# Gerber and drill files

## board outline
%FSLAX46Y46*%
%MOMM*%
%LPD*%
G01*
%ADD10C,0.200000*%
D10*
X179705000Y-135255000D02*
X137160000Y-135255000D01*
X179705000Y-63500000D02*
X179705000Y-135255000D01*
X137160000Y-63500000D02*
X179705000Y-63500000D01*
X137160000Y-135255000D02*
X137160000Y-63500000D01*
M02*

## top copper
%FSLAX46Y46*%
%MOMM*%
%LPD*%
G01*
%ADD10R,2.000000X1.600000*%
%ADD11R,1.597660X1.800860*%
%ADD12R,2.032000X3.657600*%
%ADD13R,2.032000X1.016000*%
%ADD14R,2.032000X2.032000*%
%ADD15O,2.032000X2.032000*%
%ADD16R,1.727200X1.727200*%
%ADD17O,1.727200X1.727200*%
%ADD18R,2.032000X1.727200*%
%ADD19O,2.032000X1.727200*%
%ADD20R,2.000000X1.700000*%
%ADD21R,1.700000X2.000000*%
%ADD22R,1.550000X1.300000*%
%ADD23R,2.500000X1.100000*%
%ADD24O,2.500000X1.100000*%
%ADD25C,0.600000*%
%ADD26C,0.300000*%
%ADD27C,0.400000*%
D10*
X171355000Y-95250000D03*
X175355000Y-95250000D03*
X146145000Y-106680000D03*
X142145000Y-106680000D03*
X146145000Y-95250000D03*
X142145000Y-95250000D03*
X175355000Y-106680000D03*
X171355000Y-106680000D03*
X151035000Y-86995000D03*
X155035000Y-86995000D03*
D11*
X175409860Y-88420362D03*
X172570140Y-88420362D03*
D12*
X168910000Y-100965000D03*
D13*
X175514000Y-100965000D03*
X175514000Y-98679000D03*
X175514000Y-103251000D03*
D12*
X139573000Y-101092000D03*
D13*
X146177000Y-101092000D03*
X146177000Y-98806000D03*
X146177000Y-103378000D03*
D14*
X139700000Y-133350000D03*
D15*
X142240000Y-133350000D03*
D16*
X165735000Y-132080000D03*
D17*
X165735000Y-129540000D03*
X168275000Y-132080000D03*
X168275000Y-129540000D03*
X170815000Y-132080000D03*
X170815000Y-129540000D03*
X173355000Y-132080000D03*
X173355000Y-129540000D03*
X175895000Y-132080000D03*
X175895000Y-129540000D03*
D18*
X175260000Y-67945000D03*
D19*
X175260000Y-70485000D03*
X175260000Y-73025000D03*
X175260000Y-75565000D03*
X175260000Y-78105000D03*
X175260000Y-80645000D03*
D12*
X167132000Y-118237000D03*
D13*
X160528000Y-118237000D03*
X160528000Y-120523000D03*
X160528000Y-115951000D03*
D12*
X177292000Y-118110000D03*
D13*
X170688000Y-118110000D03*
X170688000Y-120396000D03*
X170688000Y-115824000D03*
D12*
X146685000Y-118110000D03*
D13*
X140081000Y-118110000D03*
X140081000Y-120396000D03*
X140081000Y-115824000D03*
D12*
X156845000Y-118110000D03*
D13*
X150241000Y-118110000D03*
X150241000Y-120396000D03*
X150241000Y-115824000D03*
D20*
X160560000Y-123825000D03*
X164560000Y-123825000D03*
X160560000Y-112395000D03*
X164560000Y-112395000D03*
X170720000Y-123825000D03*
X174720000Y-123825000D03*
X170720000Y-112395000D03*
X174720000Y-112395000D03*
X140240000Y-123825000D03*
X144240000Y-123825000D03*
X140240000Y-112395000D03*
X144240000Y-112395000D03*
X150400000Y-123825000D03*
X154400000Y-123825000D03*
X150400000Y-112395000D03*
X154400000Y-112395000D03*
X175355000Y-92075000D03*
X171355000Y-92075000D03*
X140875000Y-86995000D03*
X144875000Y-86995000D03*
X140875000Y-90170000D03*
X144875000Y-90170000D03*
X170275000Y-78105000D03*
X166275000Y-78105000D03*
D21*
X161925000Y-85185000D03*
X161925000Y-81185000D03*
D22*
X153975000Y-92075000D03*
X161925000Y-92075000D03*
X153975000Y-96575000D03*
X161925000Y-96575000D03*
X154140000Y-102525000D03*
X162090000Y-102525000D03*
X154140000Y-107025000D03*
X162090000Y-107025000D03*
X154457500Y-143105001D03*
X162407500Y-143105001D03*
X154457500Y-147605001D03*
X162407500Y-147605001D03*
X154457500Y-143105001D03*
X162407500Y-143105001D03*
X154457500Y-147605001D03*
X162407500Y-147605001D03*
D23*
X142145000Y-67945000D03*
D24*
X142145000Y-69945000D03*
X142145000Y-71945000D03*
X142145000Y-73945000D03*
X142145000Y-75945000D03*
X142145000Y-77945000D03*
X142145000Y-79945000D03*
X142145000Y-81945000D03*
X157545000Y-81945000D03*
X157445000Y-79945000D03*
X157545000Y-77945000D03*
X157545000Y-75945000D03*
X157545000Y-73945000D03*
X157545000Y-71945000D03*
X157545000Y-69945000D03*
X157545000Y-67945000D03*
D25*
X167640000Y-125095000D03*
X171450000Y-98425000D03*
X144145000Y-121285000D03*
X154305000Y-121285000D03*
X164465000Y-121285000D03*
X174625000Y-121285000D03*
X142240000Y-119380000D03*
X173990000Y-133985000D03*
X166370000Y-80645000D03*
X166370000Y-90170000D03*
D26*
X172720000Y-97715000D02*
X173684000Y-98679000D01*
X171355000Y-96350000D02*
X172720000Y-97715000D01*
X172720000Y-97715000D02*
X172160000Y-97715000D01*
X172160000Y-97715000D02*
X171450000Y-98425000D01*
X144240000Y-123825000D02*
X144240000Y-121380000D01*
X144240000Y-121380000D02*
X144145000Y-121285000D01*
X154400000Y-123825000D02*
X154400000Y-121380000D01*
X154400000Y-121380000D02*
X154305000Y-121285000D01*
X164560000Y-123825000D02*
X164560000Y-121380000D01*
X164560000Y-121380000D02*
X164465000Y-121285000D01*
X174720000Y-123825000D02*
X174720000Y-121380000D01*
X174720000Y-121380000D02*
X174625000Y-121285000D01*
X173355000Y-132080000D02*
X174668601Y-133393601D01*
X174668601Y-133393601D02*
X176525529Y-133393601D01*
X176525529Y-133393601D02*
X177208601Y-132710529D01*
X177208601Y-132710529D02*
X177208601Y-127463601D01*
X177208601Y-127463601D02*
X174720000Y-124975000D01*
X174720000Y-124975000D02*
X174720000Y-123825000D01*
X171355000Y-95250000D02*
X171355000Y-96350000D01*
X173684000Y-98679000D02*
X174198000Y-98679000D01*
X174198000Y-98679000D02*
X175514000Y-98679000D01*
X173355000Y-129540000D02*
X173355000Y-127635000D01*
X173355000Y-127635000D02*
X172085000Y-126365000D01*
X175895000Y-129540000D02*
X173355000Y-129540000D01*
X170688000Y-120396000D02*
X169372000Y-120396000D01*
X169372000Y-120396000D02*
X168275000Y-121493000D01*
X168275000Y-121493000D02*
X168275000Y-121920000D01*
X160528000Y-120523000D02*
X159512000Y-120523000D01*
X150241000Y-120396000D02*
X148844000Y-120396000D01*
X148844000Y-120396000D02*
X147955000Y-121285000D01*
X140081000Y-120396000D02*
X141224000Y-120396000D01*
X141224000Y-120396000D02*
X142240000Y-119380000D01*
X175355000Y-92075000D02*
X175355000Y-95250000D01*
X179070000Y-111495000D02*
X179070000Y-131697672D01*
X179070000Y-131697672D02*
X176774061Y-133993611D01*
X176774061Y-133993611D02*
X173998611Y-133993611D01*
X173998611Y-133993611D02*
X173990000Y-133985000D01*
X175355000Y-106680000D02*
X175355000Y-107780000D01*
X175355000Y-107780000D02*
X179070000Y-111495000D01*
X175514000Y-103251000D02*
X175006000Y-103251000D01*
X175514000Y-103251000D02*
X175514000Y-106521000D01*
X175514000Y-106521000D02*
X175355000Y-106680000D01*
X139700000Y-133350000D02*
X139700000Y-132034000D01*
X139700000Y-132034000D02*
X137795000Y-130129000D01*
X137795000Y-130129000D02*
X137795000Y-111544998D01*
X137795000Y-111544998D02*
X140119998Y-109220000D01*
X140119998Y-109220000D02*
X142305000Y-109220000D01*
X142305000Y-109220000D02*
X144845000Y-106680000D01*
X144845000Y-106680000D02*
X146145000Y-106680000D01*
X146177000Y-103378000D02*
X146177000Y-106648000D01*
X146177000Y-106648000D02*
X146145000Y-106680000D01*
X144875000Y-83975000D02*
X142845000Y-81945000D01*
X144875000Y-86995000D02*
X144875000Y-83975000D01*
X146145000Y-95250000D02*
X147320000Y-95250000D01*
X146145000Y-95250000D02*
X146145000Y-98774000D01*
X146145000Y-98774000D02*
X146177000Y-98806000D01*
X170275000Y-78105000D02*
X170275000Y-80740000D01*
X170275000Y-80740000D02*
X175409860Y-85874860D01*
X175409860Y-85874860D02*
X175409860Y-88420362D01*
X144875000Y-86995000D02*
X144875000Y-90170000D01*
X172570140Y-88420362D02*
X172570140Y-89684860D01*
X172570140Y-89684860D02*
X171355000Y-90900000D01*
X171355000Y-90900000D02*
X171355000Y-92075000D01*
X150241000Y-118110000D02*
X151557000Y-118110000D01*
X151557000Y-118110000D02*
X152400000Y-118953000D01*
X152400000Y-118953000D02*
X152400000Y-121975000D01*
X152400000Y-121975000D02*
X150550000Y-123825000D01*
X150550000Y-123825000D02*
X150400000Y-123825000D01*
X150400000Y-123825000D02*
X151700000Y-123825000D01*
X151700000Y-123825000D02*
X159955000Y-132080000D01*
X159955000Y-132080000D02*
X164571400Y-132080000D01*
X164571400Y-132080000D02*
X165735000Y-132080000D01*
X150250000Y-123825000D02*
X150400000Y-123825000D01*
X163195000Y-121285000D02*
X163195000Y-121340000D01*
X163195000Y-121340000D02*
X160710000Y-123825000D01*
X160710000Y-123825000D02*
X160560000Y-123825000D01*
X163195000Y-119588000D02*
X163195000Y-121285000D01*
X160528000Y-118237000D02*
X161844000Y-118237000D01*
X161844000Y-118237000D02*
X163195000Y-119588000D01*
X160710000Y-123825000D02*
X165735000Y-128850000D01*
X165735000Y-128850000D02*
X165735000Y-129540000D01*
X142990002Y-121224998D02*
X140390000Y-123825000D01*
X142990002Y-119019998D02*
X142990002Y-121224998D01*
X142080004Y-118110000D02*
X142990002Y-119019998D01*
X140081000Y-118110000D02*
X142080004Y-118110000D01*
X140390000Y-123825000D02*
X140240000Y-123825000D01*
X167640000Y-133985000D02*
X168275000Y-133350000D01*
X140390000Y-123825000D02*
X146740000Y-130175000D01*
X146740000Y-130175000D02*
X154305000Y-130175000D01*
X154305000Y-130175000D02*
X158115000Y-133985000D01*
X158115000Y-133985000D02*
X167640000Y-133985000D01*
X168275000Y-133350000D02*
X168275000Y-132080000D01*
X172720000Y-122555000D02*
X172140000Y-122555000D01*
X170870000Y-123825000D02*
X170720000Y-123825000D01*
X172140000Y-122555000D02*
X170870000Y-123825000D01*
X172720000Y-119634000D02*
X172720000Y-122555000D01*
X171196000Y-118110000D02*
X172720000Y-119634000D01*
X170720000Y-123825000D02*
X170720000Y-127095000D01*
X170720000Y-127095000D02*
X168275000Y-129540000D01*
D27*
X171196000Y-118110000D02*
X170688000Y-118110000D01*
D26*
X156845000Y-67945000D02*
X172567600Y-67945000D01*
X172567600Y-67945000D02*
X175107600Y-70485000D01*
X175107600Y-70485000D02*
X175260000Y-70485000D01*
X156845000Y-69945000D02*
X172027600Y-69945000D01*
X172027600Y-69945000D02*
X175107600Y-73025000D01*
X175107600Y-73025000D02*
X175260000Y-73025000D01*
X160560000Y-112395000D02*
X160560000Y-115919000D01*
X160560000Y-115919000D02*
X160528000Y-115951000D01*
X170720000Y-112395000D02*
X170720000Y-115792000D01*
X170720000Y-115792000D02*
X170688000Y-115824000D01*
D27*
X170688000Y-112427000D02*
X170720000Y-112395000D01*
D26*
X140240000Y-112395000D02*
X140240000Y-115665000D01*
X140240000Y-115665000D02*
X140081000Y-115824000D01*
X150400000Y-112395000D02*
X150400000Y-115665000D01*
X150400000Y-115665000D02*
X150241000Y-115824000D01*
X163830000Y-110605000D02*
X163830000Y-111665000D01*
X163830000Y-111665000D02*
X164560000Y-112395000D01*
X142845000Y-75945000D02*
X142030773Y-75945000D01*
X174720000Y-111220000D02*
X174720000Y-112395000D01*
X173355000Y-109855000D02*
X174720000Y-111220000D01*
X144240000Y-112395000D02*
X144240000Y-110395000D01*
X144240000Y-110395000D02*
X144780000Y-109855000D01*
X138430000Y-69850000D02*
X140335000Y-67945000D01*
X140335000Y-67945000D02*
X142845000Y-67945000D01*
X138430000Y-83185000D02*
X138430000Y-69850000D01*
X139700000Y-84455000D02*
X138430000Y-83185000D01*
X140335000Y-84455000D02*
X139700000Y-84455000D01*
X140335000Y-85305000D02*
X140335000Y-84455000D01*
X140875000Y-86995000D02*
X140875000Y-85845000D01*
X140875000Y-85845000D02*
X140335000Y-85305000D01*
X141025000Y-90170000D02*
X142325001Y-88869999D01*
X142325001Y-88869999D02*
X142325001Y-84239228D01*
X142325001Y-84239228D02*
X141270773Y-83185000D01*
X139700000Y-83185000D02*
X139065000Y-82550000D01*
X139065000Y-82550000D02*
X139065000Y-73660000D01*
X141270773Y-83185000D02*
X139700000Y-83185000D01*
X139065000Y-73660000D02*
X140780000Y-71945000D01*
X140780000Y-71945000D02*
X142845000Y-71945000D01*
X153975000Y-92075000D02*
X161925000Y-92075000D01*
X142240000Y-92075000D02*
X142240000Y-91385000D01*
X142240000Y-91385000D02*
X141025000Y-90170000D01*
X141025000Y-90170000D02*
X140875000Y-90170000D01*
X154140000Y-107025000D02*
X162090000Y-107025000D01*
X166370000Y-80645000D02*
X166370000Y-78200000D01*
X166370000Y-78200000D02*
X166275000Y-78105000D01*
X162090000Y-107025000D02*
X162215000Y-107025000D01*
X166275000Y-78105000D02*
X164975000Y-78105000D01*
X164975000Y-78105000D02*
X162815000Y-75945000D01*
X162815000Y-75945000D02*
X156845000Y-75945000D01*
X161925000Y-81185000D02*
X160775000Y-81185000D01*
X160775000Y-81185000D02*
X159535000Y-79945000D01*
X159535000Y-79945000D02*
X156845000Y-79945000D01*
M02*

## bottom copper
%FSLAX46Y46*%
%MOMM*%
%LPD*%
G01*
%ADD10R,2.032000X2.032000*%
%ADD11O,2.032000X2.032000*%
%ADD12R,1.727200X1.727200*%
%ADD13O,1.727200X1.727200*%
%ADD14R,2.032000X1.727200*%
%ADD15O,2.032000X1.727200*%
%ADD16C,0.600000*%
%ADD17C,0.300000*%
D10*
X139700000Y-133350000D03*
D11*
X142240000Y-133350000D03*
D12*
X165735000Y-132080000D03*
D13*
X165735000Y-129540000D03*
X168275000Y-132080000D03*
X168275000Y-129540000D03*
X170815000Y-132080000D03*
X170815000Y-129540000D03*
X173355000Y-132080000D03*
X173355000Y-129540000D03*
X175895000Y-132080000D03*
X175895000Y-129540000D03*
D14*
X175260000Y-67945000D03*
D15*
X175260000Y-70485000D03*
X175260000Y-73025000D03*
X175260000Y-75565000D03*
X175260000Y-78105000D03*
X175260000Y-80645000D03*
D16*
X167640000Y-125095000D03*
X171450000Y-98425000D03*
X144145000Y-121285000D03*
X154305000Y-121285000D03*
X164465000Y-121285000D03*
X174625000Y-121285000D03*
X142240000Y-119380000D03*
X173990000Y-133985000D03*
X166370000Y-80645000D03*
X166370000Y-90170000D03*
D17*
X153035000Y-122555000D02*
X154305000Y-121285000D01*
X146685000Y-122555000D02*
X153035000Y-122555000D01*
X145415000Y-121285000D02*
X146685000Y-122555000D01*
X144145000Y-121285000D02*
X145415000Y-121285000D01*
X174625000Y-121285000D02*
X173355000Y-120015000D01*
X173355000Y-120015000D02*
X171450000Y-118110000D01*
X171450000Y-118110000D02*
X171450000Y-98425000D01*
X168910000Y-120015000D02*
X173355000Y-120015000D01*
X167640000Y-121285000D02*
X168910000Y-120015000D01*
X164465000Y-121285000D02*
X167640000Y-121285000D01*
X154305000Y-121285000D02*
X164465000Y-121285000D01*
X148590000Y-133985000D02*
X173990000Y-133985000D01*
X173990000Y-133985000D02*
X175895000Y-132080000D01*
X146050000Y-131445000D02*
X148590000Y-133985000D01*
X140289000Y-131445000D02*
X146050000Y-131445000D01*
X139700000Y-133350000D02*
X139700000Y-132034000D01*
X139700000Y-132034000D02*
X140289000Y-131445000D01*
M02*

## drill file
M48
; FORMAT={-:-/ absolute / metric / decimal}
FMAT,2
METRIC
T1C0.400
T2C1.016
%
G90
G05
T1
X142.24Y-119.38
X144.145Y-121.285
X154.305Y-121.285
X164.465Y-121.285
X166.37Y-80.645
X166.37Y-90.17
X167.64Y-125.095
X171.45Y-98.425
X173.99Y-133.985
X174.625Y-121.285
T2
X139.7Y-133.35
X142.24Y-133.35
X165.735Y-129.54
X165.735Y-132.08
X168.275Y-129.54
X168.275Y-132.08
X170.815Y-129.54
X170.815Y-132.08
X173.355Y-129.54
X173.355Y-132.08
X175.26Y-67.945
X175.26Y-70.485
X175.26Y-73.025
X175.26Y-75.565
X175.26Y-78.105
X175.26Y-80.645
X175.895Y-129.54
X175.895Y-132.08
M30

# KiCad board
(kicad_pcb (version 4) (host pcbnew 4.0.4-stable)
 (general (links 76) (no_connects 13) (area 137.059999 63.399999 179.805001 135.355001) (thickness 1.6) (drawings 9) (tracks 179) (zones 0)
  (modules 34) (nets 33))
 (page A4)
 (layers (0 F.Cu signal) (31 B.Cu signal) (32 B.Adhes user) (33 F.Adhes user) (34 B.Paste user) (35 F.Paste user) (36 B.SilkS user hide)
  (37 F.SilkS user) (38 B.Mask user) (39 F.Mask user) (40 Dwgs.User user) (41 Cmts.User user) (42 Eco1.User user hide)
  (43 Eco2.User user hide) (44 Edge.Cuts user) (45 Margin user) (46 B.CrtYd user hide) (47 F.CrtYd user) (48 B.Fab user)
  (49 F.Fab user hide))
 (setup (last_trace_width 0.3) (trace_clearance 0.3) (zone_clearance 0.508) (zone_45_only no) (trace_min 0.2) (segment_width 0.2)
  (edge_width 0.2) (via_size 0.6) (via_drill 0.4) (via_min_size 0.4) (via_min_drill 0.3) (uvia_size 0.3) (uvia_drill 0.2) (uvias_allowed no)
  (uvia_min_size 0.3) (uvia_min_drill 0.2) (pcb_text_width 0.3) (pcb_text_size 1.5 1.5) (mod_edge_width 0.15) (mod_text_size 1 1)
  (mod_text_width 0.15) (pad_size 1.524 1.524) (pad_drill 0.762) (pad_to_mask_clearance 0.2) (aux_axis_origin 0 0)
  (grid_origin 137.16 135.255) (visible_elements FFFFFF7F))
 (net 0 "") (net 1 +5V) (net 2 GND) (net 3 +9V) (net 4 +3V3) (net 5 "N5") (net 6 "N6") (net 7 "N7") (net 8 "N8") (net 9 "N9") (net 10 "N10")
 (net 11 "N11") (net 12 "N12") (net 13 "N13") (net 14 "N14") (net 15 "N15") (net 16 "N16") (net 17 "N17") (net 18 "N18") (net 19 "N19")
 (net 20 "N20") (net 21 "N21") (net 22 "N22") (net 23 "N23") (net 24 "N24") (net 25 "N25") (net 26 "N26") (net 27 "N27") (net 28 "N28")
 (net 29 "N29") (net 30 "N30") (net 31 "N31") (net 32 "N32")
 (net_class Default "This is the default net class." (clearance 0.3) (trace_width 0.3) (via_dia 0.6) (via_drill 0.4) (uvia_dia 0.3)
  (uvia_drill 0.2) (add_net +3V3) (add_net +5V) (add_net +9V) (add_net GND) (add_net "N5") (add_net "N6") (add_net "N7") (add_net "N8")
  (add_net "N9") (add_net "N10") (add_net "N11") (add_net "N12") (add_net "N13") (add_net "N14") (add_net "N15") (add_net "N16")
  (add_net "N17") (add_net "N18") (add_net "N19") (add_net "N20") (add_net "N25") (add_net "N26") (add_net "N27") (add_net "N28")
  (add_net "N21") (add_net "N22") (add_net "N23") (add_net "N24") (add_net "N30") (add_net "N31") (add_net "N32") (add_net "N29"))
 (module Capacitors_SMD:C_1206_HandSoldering (layer F.Cu) (at 173.355 95.25)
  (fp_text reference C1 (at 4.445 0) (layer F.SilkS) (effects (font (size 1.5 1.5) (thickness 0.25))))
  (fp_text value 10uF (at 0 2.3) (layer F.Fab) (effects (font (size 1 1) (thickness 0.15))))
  (pad 1 smd rect (at -2 0) (size 2 1.6) (layers F.Cu F.Paste F.Mask) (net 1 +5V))
  (pad 2 smd rect (at 2 0) (size 2 1.6) (layers F.Cu F.Paste F.Mask) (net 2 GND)))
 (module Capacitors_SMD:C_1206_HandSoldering (layer F.Cu) (at 144.145 106.68 180)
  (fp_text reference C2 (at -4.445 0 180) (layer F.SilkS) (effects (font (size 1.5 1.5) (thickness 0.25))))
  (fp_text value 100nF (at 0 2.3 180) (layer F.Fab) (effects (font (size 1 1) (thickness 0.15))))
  (pad 1 smd rect (at -2 0 180) (size 2 1.6) (layers F.Cu F.Paste F.Mask) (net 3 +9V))
  (pad 2 smd rect (at 2 0 180) (size 2 1.6) (layers F.Cu F.Paste F.Mask) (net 2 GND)))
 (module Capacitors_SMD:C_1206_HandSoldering (layer F.Cu) (at 144.145 95.25 180)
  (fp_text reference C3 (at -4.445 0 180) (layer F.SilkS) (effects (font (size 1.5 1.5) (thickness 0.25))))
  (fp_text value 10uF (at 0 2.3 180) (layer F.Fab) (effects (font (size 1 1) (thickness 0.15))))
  (pad 1 smd rect (at -2 0 180) (size 2 1.6) (layers F.Cu F.Paste F.Mask) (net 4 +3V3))
  (pad 2 smd rect (at 2 0 180) (size 2 1.6) (layers F.Cu F.Paste F.Mask) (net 2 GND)))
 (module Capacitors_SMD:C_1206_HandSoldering (layer F.Cu) (at 173.355 106.68 180)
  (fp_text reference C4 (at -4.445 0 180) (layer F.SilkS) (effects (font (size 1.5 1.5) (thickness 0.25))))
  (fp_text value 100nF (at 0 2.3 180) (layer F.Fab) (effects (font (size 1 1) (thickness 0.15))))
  (pad 1 smd rect (at -2 0 180) (size 2 1.6) (layers F.Cu F.Paste F.Mask) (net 3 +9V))
  (pad 2 smd rect (at 2 0 180) (size 2 1.6) (layers F.Cu F.Paste F.Mask) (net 2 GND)))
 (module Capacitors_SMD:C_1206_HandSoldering (layer F.Cu) (at 153.035 86.995)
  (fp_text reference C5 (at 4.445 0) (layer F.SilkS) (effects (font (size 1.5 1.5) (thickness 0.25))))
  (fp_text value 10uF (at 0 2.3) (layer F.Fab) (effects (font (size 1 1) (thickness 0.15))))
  (pad 1 smd rect (at -2 0) (size 2 1.6) (layers F.Cu F.Paste F.Mask) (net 4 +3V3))
  (pad 2 smd rect (at 2 0) (size 2 1.6) (layers F.Cu F.Paste F.Mask) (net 2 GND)))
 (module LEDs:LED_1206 (layer F.Cu) (at 173.99 88.420362)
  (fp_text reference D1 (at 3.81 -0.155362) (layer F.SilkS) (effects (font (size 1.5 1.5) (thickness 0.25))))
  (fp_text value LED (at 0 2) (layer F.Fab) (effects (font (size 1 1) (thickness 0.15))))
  (pad 2 smd rect (at 1.41986 0 180) (size 1.59766 1.80086) (layers F.Cu F.Paste F.Mask) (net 4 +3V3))
  (pad 1 smd rect (at -1.41986 0 180) (size 1.59766 1.80086) (layers F.Cu F.Paste F.Mask) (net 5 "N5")))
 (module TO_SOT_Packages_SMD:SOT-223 (layer F.Cu) (at 172.212 100.965 90)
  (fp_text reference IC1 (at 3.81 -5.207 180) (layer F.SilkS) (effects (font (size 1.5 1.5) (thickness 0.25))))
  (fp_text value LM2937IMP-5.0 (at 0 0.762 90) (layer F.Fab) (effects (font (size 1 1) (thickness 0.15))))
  (pad 4 smd rect (at 0 -3.302 90) (size 3.6576 2.032) (layers F.Cu F.Paste F.Mask) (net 2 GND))
  (pad 2 smd rect (at 0 3.302 90) (size 1.016 2.032) (layers F.Cu F.Paste F.Mask) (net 2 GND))
  (pad 3 smd rect (at 2.286 3.302 90) (size 1.016 2.032) (layers F.Cu F.Paste F.Mask) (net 1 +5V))
  (pad 1 smd rect (at -2.286 3.302 90) (size 1.016 2.032) (layers F.Cu F.Paste F.Mask) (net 3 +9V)))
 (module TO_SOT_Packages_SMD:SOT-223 (layer F.Cu) (at 142.875 101.092 90)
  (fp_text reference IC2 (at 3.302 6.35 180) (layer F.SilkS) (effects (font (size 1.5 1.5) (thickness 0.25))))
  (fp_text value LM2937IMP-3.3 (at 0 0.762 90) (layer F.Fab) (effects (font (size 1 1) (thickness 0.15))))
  (pad 4 smd rect (at 0 -3.302 90) (size 3.6576 2.032) (layers F.Cu F.Paste F.Mask) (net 2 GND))
  (pad 2 smd rect (at 0 3.302 90) (size 1.016 2.032) (layers F.Cu F.Paste F.Mask) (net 2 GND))
  (pad 3 smd rect (at 2.286 3.302 90) (size 1.016 2.032) (layers F.Cu F.Paste F.Mask) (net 4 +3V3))
  (pad 1 smd rect (at -2.286 3.302 90) (size 1.016 2.032) (layers F.Cu F.Paste F.Mask) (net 3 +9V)))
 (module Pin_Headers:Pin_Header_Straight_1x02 (layer F.Cu) (at 139.7 133.35 90)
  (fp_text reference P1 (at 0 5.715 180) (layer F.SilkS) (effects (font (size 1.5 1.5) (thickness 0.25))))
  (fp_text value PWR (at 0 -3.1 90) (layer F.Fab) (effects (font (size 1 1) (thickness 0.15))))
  (pad 1 thru_hole rect (at 0 0 90) (size 2.032 2.032) (drill 1.016) (layers *.Cu *.Mask) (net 3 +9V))
  (pad 2 thru_hole oval (at 0 2.54 90) (size 2.032 2.032) (drill 1.016) (layers *.Cu *.Mask) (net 2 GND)))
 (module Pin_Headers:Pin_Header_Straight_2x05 (layer F.Cu) (at 165.735 132.08 90)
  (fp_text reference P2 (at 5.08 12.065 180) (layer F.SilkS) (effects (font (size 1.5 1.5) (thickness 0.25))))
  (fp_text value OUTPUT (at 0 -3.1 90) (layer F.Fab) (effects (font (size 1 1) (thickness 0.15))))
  (pad 1 thru_hole rect (at 0 0 90) (size 1.7272 1.7272) (drill 1.016) (layers *.Cu *.Mask) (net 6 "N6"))
  (pad 2 thru_hole oval (at 2.54 0 90) (size 1.7272 1.7272) (drill 1.016) (layers *.Cu *.Mask) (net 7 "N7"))
  (pad 3 thru_hole oval (at 0 2.54 90) (size 1.7272 1.7272) (drill 1.016) (layers *.Cu *.Mask) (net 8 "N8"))
  (pad 4 thru_hole oval (at 2.54 2.54 90) (size 1.7272 1.7272) (drill 1.016) (layers *.Cu *.Mask) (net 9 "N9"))
  (pad 5 thru_hole oval (at 0 5.08 90) (size 1.7272 1.7272) (drill 1.016) (layers *.Cu *.Mask) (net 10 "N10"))
  (pad 6 thru_hole oval (at 2.54 5.08 90) (size 1.7272 1.7272) (drill 1.016) (layers *.Cu *.Mask) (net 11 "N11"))
  (pad 7 thru_hole oval (at 0 7.62 90) (size 1.7272 1.7272) (drill 1.016) (layers *.Cu *.Mask) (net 1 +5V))
  (pad 8 thru_hole oval (at 2.54 7.62 90) (size 1.7272 1.7272) (drill 1.016) (layers *.Cu *.Mask) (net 2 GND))
  (pad 9 thru_hole oval (at 0 10.16 90) (size 1.7272 1.7272) (drill 1.016) (layers *.Cu *.Mask) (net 3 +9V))
  (pad 10 thru_hole oval (at 2.54 10.16 90) (size 1.7272 1.7272) (drill 1.016) (layers *.Cu *.Mask) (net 2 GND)))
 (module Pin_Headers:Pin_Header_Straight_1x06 (layer F.Cu) (at 175.26 67.945)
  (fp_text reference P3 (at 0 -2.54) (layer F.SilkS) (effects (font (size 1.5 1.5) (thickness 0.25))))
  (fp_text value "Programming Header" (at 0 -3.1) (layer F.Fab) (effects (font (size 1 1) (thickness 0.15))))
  (pad 1 thru_hole rect (at 0 0) (size 2.032 1.7272) (drill 1.016) (layers *.Cu *.Mask) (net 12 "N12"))
  (pad 2 thru_hole oval (at 0 2.54) (size 2.032 1.7272) (drill 1.016) (layers *.Cu *.Mask) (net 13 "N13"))
  (pad 3 thru_hole oval (at 0 5.08) (size 2.032 1.7272) (drill 1.016) (layers *.Cu *.Mask) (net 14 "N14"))
  (pad 4 thru_hole oval (at 0 7.62) (size 2.032 1.7272) (drill 1.016) (layers *.Cu *.Mask) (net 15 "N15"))
  (pad 5 thru_hole oval (at 0 10.16) (size 2.032 1.7272) (drill 1.016) (layers *.Cu *.Mask) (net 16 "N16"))
  (pad 6 thru_hole oval (at 0 12.7) (size 2.032 1.7272) (drill 1.016) (layers *.Cu *.Mask) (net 2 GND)))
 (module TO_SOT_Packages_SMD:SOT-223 (layer F.Cu) (at 163.83 118.237 270)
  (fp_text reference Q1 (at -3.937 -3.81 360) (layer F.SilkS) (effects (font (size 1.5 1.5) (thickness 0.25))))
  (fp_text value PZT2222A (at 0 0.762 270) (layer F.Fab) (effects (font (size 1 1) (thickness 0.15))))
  (pad 4 smd rect (at 0 -3.302 270) (size 3.6576 2.032) (layers F.Cu F.Paste F.Mask))
  (pad 2 smd rect (at 0 3.302 270) (size 1.016 2.032) (layers F.Cu F.Paste F.Mask) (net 7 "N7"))
  (pad 3 smd rect (at 2.286 3.302 270) (size 1.016 2.032) (layers F.Cu F.Paste F.Mask) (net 2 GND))
  (pad 1 smd rect (at -2.286 3.302 270) (size 1.016 2.032) (layers F.Cu F.Paste F.Mask) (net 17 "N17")))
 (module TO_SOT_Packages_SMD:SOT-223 (layer F.Cu) (at 173.99 118.11 270)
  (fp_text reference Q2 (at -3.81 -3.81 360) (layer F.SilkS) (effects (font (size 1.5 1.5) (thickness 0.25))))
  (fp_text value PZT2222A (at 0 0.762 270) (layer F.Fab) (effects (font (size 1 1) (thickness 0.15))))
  (pad 4 smd rect (at 0 -3.302 270) (size 3.6576 2.032) (layers F.Cu F.Paste F.Mask))
  (pad 2 smd rect (at 0 3.302 270) (size 1.016 2.032) (layers F.Cu F.Paste F.Mask) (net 9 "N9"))
  (pad 3 smd rect (at 2.286 3.302 270) (size 1.016 2.032) (layers F.Cu F.Paste F.Mask) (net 2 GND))
  (pad 1 smd rect (at -2.286 3.302 270) (size 1.016 2.032) (layers F.Cu F.Paste F.Mask) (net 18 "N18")))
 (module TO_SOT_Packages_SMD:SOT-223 (layer F.Cu) (at 143.383 118.11 270)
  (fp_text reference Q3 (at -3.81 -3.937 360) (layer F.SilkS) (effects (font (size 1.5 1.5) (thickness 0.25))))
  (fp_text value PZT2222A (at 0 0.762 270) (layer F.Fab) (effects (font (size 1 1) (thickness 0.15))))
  (pad 4 smd rect (at 0 -3.302 270) (size 3.6576 2.032) (layers F.Cu F.Paste F.Mask))
  (pad 2 smd rect (at 0 3.302 270) (size 1.016 2.032) (layers F.Cu F.Paste F.Mask) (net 8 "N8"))
  (pad 3 smd rect (at 2.286 3.302 270) (size 1.016 2.032) (layers F.Cu F.Paste F.Mask) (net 2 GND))
  (pad 1 smd rect (at -2.286 3.302 270) (size 1.016 2.032) (layers F.Cu F.Paste F.Mask) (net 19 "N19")))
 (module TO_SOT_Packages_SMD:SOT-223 (layer F.Cu) (at 153.543 118.11 270)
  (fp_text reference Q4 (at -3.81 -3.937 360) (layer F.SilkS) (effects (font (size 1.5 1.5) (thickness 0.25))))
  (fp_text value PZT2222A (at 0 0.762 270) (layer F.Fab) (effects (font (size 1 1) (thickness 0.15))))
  (pad 4 smd rect (at 0 -3.302 270) (size 3.6576 2.032) (layers F.Cu F.Paste F.Mask))
  (pad 2 smd rect (at 0 3.302 270) (size 1.016 2.032) (layers F.Cu F.Paste F.Mask) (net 6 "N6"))
  (pad 3 smd rect (at 2.286 3.302 270) (size 1.016 2.032) (layers F.Cu F.Paste F.Mask) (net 2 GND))
  (pad 1 smd rect (at -2.286 3.302 270) (size 1.016 2.032) (layers F.Cu F.Paste F.Mask) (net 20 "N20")))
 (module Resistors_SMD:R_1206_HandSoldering (layer F.Cu) (at 162.56 123.825)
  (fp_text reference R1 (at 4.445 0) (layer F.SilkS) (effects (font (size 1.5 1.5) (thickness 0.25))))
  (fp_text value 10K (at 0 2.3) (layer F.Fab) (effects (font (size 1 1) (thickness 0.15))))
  (pad 1 smd rect (at -2 0) (size 2 1.7) (layers F.Cu F.Paste F.Mask) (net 7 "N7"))
  (pad 2 smd rect (at 2 0) (size 2 1.7) (layers F.Cu F.Paste F.Mask) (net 1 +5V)))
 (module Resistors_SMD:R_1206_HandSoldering (layer F.Cu) (at 162.56 112.395)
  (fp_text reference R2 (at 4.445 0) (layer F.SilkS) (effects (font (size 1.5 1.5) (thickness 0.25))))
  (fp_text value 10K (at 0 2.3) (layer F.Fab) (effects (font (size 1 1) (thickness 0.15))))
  (pad 1 smd rect (at -2 0) (size 2 1.7) (layers F.Cu F.Paste F.Mask) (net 17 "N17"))
  (pad 2 smd rect (at 2 0) (size 2 1.7) (layers F.Cu F.Paste F.Mask) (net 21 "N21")))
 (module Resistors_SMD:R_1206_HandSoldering (layer F.Cu) (at 172.72 123.825)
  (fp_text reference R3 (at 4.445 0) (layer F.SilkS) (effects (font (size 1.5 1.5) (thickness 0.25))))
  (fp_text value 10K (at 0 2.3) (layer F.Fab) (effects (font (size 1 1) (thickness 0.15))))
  (pad 1 smd rect (at -2 0) (size 2 1.7) (layers F.Cu F.Paste F.Mask) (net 9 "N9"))
  (pad 2 smd rect (at 2 0) (size 2 1.7) (layers F.Cu F.Paste F.Mask) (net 1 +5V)))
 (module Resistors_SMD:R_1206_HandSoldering (layer F.Cu) (at 172.72 112.395)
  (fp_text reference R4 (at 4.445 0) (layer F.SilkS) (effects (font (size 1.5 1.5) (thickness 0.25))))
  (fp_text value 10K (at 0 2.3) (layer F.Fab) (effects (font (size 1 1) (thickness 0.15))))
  (pad 1 smd rect (at -2 0) (size 2 1.7) (layers F.Cu F.Paste F.Mask) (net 18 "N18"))
  (pad 2 smd rect (at 2 0) (size 2 1.7) (layers F.Cu F.Paste F.Mask) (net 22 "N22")))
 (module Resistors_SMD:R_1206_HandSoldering (layer F.Cu) (at 142.24 123.825)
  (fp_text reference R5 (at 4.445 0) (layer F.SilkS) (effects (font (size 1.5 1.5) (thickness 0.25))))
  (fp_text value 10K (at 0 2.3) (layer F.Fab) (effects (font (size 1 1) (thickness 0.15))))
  (pad 1 smd rect (at -2 0) (size 2 1.7) (layers F.Cu F.Paste F.Mask) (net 8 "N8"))
  (pad 2 smd rect (at 2 0) (size 2 1.7) (layers F.Cu F.Paste F.Mask) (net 1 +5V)))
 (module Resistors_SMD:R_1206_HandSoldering (layer F.Cu) (at 142.24 112.395)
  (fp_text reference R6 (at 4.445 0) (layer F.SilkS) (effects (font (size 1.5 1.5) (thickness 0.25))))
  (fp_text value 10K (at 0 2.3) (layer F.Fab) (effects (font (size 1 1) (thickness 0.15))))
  (pad 1 smd rect (at -2 0) (size 2 1.7) (layers F.Cu F.Paste F.Mask) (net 19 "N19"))
  (pad 2 smd rect (at 2 0) (size 2 1.7) (layers F.Cu F.Paste F.Mask) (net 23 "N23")))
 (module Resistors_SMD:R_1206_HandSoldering (layer F.Cu) (at 152.4 123.825)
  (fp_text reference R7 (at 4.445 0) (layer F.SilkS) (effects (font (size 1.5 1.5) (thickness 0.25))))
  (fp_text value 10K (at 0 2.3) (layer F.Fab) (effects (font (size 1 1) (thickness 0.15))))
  (pad 1 smd rect (at -2 0) (size 2 1.7) (layers F.Cu F.Paste F.Mask) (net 6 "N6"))
  (pad 2 smd rect (at 2 0) (size 2 1.7) (layers F.Cu F.Paste F.Mask) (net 1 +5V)))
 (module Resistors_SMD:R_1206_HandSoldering (layer F.Cu) (at 152.4 112.395)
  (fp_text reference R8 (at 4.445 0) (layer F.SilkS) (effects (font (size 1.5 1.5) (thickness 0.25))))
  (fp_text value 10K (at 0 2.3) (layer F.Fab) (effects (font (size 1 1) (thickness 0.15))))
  (pad 1 smd rect (at -2 0) (size 2 1.7) (layers F.Cu F.Paste F.Mask) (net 20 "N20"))
  (pad 2 smd rect (at 2 0) (size 2 1.7) (layers F.Cu F.Paste F.Mask) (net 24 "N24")))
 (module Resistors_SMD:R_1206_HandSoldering (layer F.Cu) (at 173.355 92.075 180)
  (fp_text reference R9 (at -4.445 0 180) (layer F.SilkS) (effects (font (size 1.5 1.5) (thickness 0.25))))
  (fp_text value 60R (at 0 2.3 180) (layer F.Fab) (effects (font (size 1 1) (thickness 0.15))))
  (pad 1 smd rect (at -2 0 180) (size 2 1.7) (layers F.Cu F.Paste F.Mask) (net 2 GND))
  (pad 2 smd rect (at 2 0 180) (size 2 1.7) (layers F.Cu F.Paste F.Mask) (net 5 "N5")))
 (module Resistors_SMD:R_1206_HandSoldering (layer F.Cu) (at 142.875 86.995)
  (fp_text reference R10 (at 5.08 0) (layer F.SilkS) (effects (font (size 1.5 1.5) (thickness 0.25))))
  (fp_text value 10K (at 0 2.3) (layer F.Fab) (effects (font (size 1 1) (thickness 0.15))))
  (pad 1 smd rect (at -2 0) (size 2 1.7) (layers F.Cu F.Paste F.Mask) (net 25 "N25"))
  (pad 2 smd rect (at 2 0) (size 2 1.7) (layers F.Cu F.Paste F.Mask) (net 4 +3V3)))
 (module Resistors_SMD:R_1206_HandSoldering (layer F.Cu) (at 142.875 90.17)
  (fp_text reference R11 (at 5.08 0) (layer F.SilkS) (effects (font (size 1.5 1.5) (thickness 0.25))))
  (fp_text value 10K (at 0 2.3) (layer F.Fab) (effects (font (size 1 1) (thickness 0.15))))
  (pad 1 smd rect (at -2 0) (size 2 1.7) (layers F.Cu F.Paste F.Mask) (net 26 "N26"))
  (pad 2 smd rect (at 2 0) (size 2 1.7) (layers F.Cu F.Paste F.Mask) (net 4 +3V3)))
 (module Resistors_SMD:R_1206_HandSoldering (layer F.Cu) (at 168.275 78.105 180)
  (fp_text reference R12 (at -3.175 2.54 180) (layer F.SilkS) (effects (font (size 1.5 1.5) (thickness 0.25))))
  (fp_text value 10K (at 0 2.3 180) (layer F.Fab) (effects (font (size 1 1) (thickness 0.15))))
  (pad 1 smd rect (at -2 0 180) (size 2 1.7) (layers F.Cu F.Paste F.Mask) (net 4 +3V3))
  (pad 2 smd rect (at 2 0 180) (size 2 1.7) (layers F.Cu F.Paste F.Mask) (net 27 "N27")))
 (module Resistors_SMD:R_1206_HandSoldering (layer F.Cu) (at 161.925 83.185 90)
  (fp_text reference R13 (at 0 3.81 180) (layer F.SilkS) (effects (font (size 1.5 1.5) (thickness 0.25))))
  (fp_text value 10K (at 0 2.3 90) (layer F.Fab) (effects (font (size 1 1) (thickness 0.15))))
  (pad 1 smd rect (at -2 0 90) (size 2 1.7) (layers F.Cu F.Paste F.Mask) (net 2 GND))
  (pad 2 smd rect (at 2 0 90) (size 2 1.7) (layers F.Cu F.Paste F.Mask) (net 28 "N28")))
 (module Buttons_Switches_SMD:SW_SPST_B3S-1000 (layer F.Cu) (at 157.95 94.325)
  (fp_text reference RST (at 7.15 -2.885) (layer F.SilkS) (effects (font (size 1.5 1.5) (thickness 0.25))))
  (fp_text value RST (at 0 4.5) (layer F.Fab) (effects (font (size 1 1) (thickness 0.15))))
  (pad 1 smd rect (at -3.975 -2.25) (size 1.55 1.3) (layers F.Cu F.Paste F.Mask) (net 26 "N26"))
  (pad 1 smd rect (at 3.975 -2.25) (size 1.55 1.3) (layers F.Cu F.Paste F.Mask) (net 26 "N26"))
  (pad 2 smd rect (at -3.975 2.25) (size 1.55 1.3) (layers F.Cu F.Paste F.Mask) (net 2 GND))
  (pad 2 smd rect (at 3.975 2.25) (size 1.55 1.3) (layers F.Cu F.Paste F.Mask) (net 2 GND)))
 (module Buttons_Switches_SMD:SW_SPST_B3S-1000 (layer F.Cu) (at 158.115 104.775)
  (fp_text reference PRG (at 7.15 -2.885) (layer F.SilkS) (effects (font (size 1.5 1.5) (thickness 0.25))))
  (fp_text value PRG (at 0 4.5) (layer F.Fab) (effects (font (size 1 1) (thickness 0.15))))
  (pad 1 smd rect (at -3.975 -2.25) (size 1.55 1.3) (layers F.Cu F.Paste F.Mask) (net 2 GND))
  (pad 1 smd rect (at 3.975 -2.25) (size 1.55 1.3) (layers F.Cu F.Paste F.Mask) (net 2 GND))
  (pad 2 smd rect (at -3.975 2.25) (size 1.55 1.3) (layers F.Cu F.Paste F.Mask) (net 27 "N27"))
  (pad 2 smd rect (at 3.975 2.25) (size 1.55 1.3) (layers F.Cu F.Paste F.Mask) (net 27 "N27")))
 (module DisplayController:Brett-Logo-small (layer B.Cu) (at 165.735 119.38 270)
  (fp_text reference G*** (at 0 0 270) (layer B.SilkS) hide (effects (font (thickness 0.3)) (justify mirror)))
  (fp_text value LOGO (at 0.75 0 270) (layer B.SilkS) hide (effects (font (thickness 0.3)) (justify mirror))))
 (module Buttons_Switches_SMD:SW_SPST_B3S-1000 (layer F.Cu) (at 158.4325 145.355001)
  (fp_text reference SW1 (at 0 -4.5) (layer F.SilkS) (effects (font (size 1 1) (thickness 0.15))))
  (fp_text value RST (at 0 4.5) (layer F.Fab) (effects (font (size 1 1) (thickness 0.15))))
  (pad 1 smd rect (at -3.975 -2.25) (size 1.55 1.3) (layers F.Cu F.Paste F.Mask) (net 26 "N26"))
  (pad 1 smd rect (at 3.975 -2.25) (size 1.55 1.3) (layers F.Cu F.Paste F.Mask) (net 26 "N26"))
  (pad 2 smd rect (at -3.975 2.25) (size 1.55 1.3) (layers F.Cu F.Paste F.Mask) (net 2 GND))
  (pad 2 smd rect (at 3.975 2.25) (size 1.55 1.3) (layers F.Cu F.Paste F.Mask) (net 2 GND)))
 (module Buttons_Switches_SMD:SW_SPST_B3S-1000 (layer F.Cu) (at 158.4325 145.355001)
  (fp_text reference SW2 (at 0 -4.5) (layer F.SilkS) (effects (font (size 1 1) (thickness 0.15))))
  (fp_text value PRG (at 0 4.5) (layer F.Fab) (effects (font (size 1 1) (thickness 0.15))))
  (pad 1 smd rect (at -3.975 -2.25) (size 1.55 1.3) (layers F.Cu F.Paste F.Mask) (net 2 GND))
  (pad 1 smd rect (at 3.975 -2.25) (size 1.55 1.3) (layers F.Cu F.Paste F.Mask) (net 2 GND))
  (pad 2 smd rect (at -3.975 2.25) (size 1.55 1.3) (layers F.Cu F.Paste F.Mask) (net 27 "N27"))
  (pad 2 smd rect (at 3.975 2.25) (size 1.55 1.3) (layers F.Cu F.Paste F.Mask) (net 27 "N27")))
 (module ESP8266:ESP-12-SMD (layer F.Cu) (at 142.845 67.945)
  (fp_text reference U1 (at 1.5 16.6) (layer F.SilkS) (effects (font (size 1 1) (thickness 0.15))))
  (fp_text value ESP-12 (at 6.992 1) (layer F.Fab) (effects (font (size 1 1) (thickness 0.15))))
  (pad 1 smd rect (at 0 0) (size 2.5 1.1) (drill (offset -0.7 0)) (layers F.Cu F.Paste F.Mask) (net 25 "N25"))
  (pad 2 smd oval (at 0 2) (size 2.5 1.1) (drill (offset -0.7 0)) (layers F.Cu F.Paste F.Mask) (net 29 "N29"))
  (pad 3 smd oval (at 0 4) (size 2.5 1.1) (drill (offset -0.7 0)) (layers F.Cu F.Paste F.Mask) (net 26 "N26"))
  (pad 4 smd oval (at 0 6) (size 2.5 1.1) (drill (offset -0.7 0)) (layers F.Cu F.Paste F.Mask) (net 21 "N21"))
  (pad 5 smd oval (at 0 8) (size 2.5 1.1) (drill (offset -0.7 0)) (layers F.Cu F.Paste F.Mask) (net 22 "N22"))
  (pad 6 smd oval (at 0 10) (size 2.5 1.1) (drill (offset -0.7 0)) (layers F.Cu F.Paste F.Mask) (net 23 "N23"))
  (pad 7 smd oval (at 0 12) (size 2.5 1.1) (drill (offset -0.7 0)) (layers F.Cu F.Paste F.Mask) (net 24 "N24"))
  (pad 8 smd oval (at 0 14) (size 2.5 1.1) (drill (offset -0.7 0)) (layers F.Cu F.Paste F.Mask) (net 4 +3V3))
  (pad 9 smd oval (at 14 14) (size 2.5 1.1) (drill (offset 0.7 0)) (layers F.Cu F.Paste F.Mask) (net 2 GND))
  (pad 10 smd oval (at 14 12) (size 2.5 1.1) (drill (offset 0.6 0)) (layers F.Cu F.Paste F.Mask) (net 28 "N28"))
  (pad 11 smd oval (at 14 10) (size 2.5 1.1) (drill (offset 0.7 0)) (layers F.Cu F.Paste F.Mask) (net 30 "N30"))
  (pad 12 smd oval (at 14 8) (size 2.5 1.1) (drill (offset 0.7 0)) (layers F.Cu F.Paste F.Mask) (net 27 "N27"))
  (pad 13 smd oval (at 14 6) (size 2.5 1.1) (drill (offset 0.7 0)) (layers F.Cu F.Paste F.Mask) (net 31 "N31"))
  (pad 14 smd oval (at 14 4) (size 2.5 1.1) (drill (offset 0.7 0)) (layers F.Cu F.Paste F.Mask) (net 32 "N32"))
  (pad 15 smd oval (at 14 2) (size 2.5 1.1) (drill (offset 0.7 0)) (layers F.Cu F.Paste F.Mask) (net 14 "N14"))
  (pad 16 smd oval (at 14 0) (size 2.5 1.1) (drill (offset 0.7 0)) (layers F.Cu F.Paste F.Mask) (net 13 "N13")))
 (gr_line (start 179.705 135.255) (end 137.16 135.255) (layer Edge.Cuts) (width 0.2))
 (gr_line (start 179.705 63.5) (end 179.705 135.255) (layer Edge.Cuts) (width 0.2))
 (gr_line (start 137.16 63.5) (end 179.705 63.5) (layer Edge.Cuts) (width 0.2))
 (gr_line (start 137.16 135.255) (end 137.16 63.5) (layer Edge.Cuts) (width 0.2))
 (via (at 167.64 125.095) (size 0.6) (drill 0.4) (layers F.Cu B.Cu) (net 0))
 (segment (start 153.035 122.555) (end 154.305 121.285) (width 0.3) (layer B.Cu) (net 1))
 (segment (start 146.685 122.555) (end 153.035 122.555) (width 0.3) (layer B.Cu) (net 1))
 (segment (start 145.415 121.285) (end 146.685 122.555) (width 0.3) (layer B.Cu) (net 1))
 (segment (start 144.145 121.285) (end 145.415 121.285) (width 0.3) (layer B.Cu) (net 1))
 (segment (start 174.625 121.285) (end 173.355 120.015) (width 0.3) (layer B.Cu) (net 1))
 (segment (start 173.355 120.015) (end 171.45 118.11) (width 0.3) (layer B.Cu) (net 1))
 (segment (start 171.45 118.11) (end 171.45 98.425) (width 0.3) (layer B.Cu) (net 1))
 (segment (start 168.91 120.015) (end 173.355 120.015) (width 0.3) (layer B.Cu) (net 1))
 (segment (start 167.64 121.285) (end 168.91 120.015) (width 0.3) (layer B.Cu) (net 1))
 (segment (start 164.465 121.285) (end 167.64 121.285) (width 0.3) (layer B.Cu) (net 1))
 (segment (start 154.305 121.285) (end 164.465 121.285) (width 0.3) (layer B.Cu) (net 1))
 (segment (start 172.72 97.715) (end 173.684 98.679) (width 0.3) (layer F.Cu) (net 1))
 (segment (start 171.355 96.35) (end 172.72 97.715) (width 0.3) (layer F.Cu) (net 1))
 (segment (start 172.72 97.715) (end 172.16 97.715) (width 0.3) (layer F.Cu) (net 1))
 (segment (start 172.16 97.715) (end 171.45 98.425) (width 0.3) (layer F.Cu) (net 1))
 (via (at 171.45 98.425) (size 0.6) (drill 0.4) (layers F.Cu B.Cu) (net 1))
 (segment (start 144.24 123.825) (end 144.24 121.38) (width 0.3) (layer F.Cu) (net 1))
 (segment (start 144.24 121.38) (end 144.145 121.285) (width 0.3) (layer F.Cu) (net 1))
 (via (at 144.145 121.285) (size 0.6) (drill 0.4) (layers F.Cu B.Cu) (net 1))
 (segment (start 154.4 123.825) (end 154.4 121.38) (width 0.3) (layer F.Cu) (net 1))
 (segment (start 154.4 121.38) (end 154.305 121.285) (width 0.3) (layer F.Cu) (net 1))
 (via (at 154.305 121.285) (size 0.6) (drill 0.4) (layers F.Cu B.Cu) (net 1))
 (segment (start 164.56 123.825) (end 164.56 121.38) (width 0.3) (layer F.Cu) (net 1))
 (segment (start 164.56 121.38) (end 164.465 121.285) (width 0.3) (layer F.Cu) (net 1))
 (via (at 164.465 121.285) (size 0.6) (drill 0.4) (layers F.Cu B.Cu) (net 1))
 (segment (start 174.72 123.825) (end 174.72 121.38) (width 0.3) (layer F.Cu) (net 1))
 (segment (start 174.72 121.38) (end 174.625 121.285) (width 0.3) (layer F.Cu) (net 1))
 (via (at 174.625 121.285) (size 0.6) (drill 0.4) (layers F.Cu B.Cu) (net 1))
 (segment (start 173.355 132.08) (end 174.668601 133.393601) (width 0.3) (layer F.Cu) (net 1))
 (segment (start 174.668601 133.393601) (end 176.525529 133.393601) (width 0.3) (layer F.Cu) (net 1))
 (segment (start 176.525529 133.393601) (end 177.208601 132.710529) (width 0.3) (layer F.Cu) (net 1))
 (segment (start 177.208601 132.710529) (end 177.208601 127.463601) (width 0.3) (layer F.Cu) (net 1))
 (segment (start 177.208601 127.463601) (end 174.72 124.975) (width 0.3) (layer F.Cu) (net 1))
 (segment (start 174.72 124.975) (end 174.72 123.825) (width 0.3) (layer F.Cu) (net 1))
 (segment (start 171.355 95.25) (end 171.355 96.35) (width 0.3) (layer F.Cu) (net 1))
 (segment (start 173.684 98.679) (end 174.198 98.679) (width 0.3) (layer F.Cu) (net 1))
 (segment (start 174.198 98.679) (end 175.514 98.679) (width 0.3) (layer F.Cu) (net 1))
 (via (at 142.24 119.38) (size 0.6) (drill 0.4) (layers F.Cu B.Cu) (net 2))
 (segment (start 173.355 129.54) (end 173.355 127.635) (width 0.3) (layer F.Cu) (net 2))
 (segment (start 173.355 127.635) (end 172.085 126.365) (width 0.3) (layer F.Cu) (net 2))
 (segment (start 175.895 129.54) (end 173.355 129.54) (width 0.3) (layer F.Cu) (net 2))
 (segment (start 170.688 120.396) (end 169.372 120.396) (width 0.3) (layer F.Cu) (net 2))
 (segment (start 169.372 120.396) (end 168.275 121.493) (width 0.3) (layer F.Cu) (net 2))
 (segment (start 168.275 121.493) (end 168.275 121.92) (width 0.3) (layer F.Cu) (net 2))
 (segment (start 160.528 120.523) (end 159.512 120.523) (width 0.3) (layer F.Cu) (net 2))
 (segment (start 150.241 120.396) (end 148.844 120.396) (width 0.3) (layer F.Cu) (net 2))
 (segment (start 148.844 120.396) (end 147.955 121.285) (width 0.3) (layer F.Cu) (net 2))
 (segment (start 140.081 120.396) (end 141.224 120.396) (width 0.3) (layer F.Cu) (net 2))
 (segment (start 141.224 120.396) (end 142.24 119.38) (width 0.3) (layer F.Cu) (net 2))
 (segment (start 175.355 92.075) (end 175.355 95.25) (width 0.3) (layer F.Cu) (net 2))
 (segment (start 179.07 111.495) (end 179.07 131.697672) (width 0.3) (layer F.Cu) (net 3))
 (segment (start 179.07 131.697672) (end 176.774061 133.993611) (width 0.3) (layer F.Cu) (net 3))
 (segment (start 176.774061 133.993611) (end 173.998611 133.993611) (width 0.3) (layer F.Cu) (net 3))
 (segment (start 173.998611 133.993611) (end 173.99 133.985) (width 0.3) (layer F.Cu) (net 3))
 (via (at 173.99 133.985) (size 0.6) (drill 0.4) (layers F.Cu B.Cu) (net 3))
 (segment (start 175.355 106.68) (end 175.355 107.78) (width 0.3) (layer F.Cu) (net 3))
 (segment (start 175.355 107.78) (end 179.07 111.495) (width 0.3) (layer F.Cu) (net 3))
 (segment (start 175.514 103.251) (end 175.006 103.251) (width 0.3) (layer F.Cu) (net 3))
 (segment (start 175.514 103.251) (end 175.514 106.521) (width 0.3) (layer F.Cu) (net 3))
 (segment (start 175.514 106.521) (end 175.355 106.68) (width 0.3) (layer F.Cu) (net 3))
 (segment (start 139.7 133.35) (end 139.7 132.034) (width 0.3) (layer F.Cu) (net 3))
 (segment (start 139.7 132.034) (end 137.795 130.129) (width 0.3) (layer F.Cu) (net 3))
 (segment (start 137.795 130.129) (end 137.795 111.544998) (width 0.3) (layer F.Cu) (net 3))
 (segment (start 137.795 111.544998) (end 140.119998 109.22) (width 0.3) (layer F.Cu) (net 3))
 (segment (start 140.119998 109.22) (end 142.305 109.22) (width 0.3) (layer F.Cu) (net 3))
 (segment (start 142.305 109.22) (end 144.845 106.68) (width 0.3) (layer F.Cu) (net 3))
 (segment (start 144.845 106.68) (end 146.145 106.68) (width 0.3) (layer F.Cu) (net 3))
 (segment (start 148.59 133.985) (end 173.99 133.985) (width 0.3) (layer B.Cu) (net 3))
 (segment (start 173.99 133.985) (end 175.895 132.08) (width 0.3) (layer B.Cu) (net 3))
 (segment (start 146.05 131.445) (end 148.59 133.985) (width 0.3) (layer B.Cu) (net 3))
 (segment (start 140.289 131.445) (end 146.05 131.445) (width 0.3) (layer B.Cu) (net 3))
 (segment (start 139.7 133.35) (end 139.7 132.034) (width 0.3) (layer B.Cu) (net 3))
 (segment (start 139.7 132.034) (end 140.289 131.445) (width 0.3) (layer B.Cu) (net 3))
 (segment (start 146.177 103.378) (end 146.177 106.648) (width 0.3) (layer F.Cu) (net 3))
 (segment (start 146.177 106.648) (end 146.145 106.68) (width 0.3) (layer F.Cu) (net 3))
 (segment (start 144.875 83.975) (end 142.845 81.945) (width 0.3) (layer F.Cu) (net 4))
 (segment (start 144.875 86.995) (end 144.875 83.975) (width 0.3) (layer F.Cu) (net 4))
 (segment (start 146.145 95.25) (end 147.32 95.25) (width 0.3) (layer F.Cu) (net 4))
 (segment (start 146.145 95.25) (end 146.145 98.774) (width 0.3) (layer F.Cu) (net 4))
 (segment (start 146.145 98.774) (end 146.177 98.806) (width 0.3) (layer F.Cu) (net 4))
 (segment (start 170.275 78.105) (end 170.275 80.74) (width 0.3) (layer F.Cu) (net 4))
 (segment (start 170.275 80.74) (end 175.40986 85.87486) (width 0.3) (layer F.Cu) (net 4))
 (segment (start 175.40986 85.87486) (end 175.40986 88.420362) (width 0.3) (layer F.Cu) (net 4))
 (segment (start 144.875 86.995) (end 144.875 90.17) (width 0.3) (layer F.Cu) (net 4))
 (segment (start 172.57014 88.420362) (end 172.57014 89.68486) (width 0.3) (layer F.Cu) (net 5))
 (segment (start 172.57014 89.68486) (end 171.355 90.9) (width 0.3) (layer F.Cu) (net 5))
 (segment (start 171.355 90.9) (end 171.355 92.075) (width 0.3) (layer F.Cu) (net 5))
 (segment (start 150.241 118.11) (end 151.557 118.11) (width 0.3) (layer F.Cu) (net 6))
 (segment (start 151.557 118.11) (end 152.4 118.953) (width 0.3) (layer F.Cu) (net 6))
 (segment (start 152.4 118.953) (end 152.4 121.975) (width 0.3) (layer F.Cu) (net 6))
 (segment (start 152.4 121.975) (end 150.55 123.825) (width 0.3) (layer F.Cu) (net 6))
 (segment (start 150.55 123.825) (end 150.4 123.825) (width 0.3) (layer F.Cu) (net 6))
 (segment (start 150.4 123.825) (end 151.7 123.825) (width 0.3) (layer F.Cu) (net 6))
 (segment (start 151.7 123.825) (end 159.955 132.08) (width 0.3) (layer F.Cu) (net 6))
 (segment (start 159.955 132.08) (end 164.5714 132.08) (width 0.3) (layer F.Cu) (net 6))
 (segment (start 164.5714 132.08) (end 165.735 132.08) (width 0.3) (layer F.Cu) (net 6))
 (segment (start 150.25 123.825) (end 150.4 123.825) (width 0.3) (layer F.Cu) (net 6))
 (segment (start 163.195 121.285) (end 163.195 121.34) (width 0.3) (layer F.Cu) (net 7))
 (segment (start 163.195 121.34) (end 160.71 123.825) (width 0.3) (layer F.Cu) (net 7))
 (segment (start 160.71 123.825) (end 160.56 123.825) (width 0.3) (layer F.Cu) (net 7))
 (segment (start 163.195 119.588) (end 163.195 121.285) (width 0.3) (layer F.Cu) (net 7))
 (segment (start 160.528 118.237) (end 161.844 118.237) (width 0.3) (layer F.Cu) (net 7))
 (segment (start 161.844 118.237) (end 163.195 119.588) (width 0.3) (layer F.Cu) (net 7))
 (segment (start 160.71 123.825) (end 165.735 128.85) (width 0.3) (layer F.Cu) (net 7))
 (segment (start 165.735 128.85) (end 165.735 129.54) (width 0.3) (layer F.Cu) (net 7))
 (segment (start 142.990002 121.224998) (end 140.39 123.825) (width 0.3) (layer F.Cu) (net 8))
 (segment (start 142.990002 119.019998) (end 142.990002 121.224998) (width 0.3) (layer F.Cu) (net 8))
 (segment (start 142.080004 118.11) (end 142.990002 119.019998) (width 0.3) (layer F.Cu) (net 8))
 (segment (start 140.081 118.11) (end 142.080004 118.11) (width 0.3) (layer F.Cu) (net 8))
 (segment (start 140.39 123.825) (end 140.24 123.825) (width 0.3) (layer F.Cu) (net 8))
 (segment (start 167.64 133.985) (end 168.275 133.35) (width 0.3) (layer F.Cu) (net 8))
 (segment (start 140.39 123.825) (end 146.74 130.175) (width 0.3) (layer F.Cu) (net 8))
 (segment (start 146.74 130.175) (end 154.305 130.175) (width 0.3) (layer F.Cu) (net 8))
 (segment (start 154.305 130.175) (end 158.115 133.985) (width 0.3) (layer F.Cu) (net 8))
 (segment (start 158.115 133.985) (end 167.64 133.985) (width 0.3) (layer F.Cu) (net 8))
 (segment (start 168.275 133.35) (end 168.275 132.08) (width 0.3) (layer F.Cu) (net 8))
 (segment (start 172.72 122.555) (end 172.14 122.555) (width 0.3) (layer F.Cu) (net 9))
 (segment (start 170.87 123.825) (end 170.72 123.825) (width 0.3) (layer F.Cu) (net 9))
 (segment (start 172.14 122.555) (end 170.87 123.825) (width 0.3) (layer F.Cu) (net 9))
 (segment (start 172.72 119.634) (end 172.72 122.555) (width 0.3) (layer F.Cu) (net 9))
 (segment (start 171.196 118.11) (end 172.72 119.634) (width 0.3) (layer F.Cu) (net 9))
 (segment (start 170.72 123.825) (end 170.72 127.095) (width 0.3) (layer F.Cu) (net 9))
 (segment (start 170.72 127.095) (end 168.275 129.54) (width 0.3) (layer F.Cu) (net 9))
 (segment (start 171.196 118.11) (end 170.688 118.11) (width 0.4) (layer F.Cu) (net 9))
 (segment (start 156.845 67.945) (end 172.5676 67.945) (width 0.3) (layer F.Cu) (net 13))
 (segment (start 172.5676 67.945) (end 175.1076 70.485) (width 0.3) (layer F.Cu) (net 13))
 (segment (start 175.1076 70.485) (end 175.26 70.485) (width 0.3) (layer F.Cu) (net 13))
 (segment (start 156.845 69.945) (end 172.0276 69.945) (width 0.3) (layer F.Cu) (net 14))
 (segment (start 172.0276 69.945) (end 175.1076 73.025) (width 0.3) (layer F.Cu) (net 14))
 (segment (start 175.1076 73.025) (end 175.26 73.025) (width 0.3) (layer F.Cu) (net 14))
 (segment (start 160.56 112.395) (end 160.56 115.919) (width 0.3) (layer F.Cu) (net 17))
 (segment (start 160.56 115.919) (end 160.528 115.951) (width 0.3) (layer F.Cu) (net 17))
 (segment (start 170.72 112.395) (end 170.72 115.792) (width 0.3) (layer F.Cu) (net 18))
 (segment (start 170.72 115.792) (end 170.688 115.824) (width 0.3) (layer F.Cu) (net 18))
 (segment (start 170.688 112.427) (end 170.72 112.395) (width 0.4) (layer F.Cu) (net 18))
 (segment (start 140.24 112.395) (end 140.24 115.665) (width 0.3) (layer F.Cu) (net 19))
 (segment (start 140.24 115.665) (end 140.081 115.824) (width 0.3) (layer F.Cu) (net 19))
 (segment (start 150.4 112.395) (end 150.4 115.665) (width 0.3) (layer F.Cu) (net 20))
 (segment (start 150.4 115.665) (end 150.241 115.824) (width 0.3) (layer F.Cu) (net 20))
 (segment (start 163.83 110.605) (end 163.83 111.665) (width 0.3) (layer F.Cu) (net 21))
 (segment (start 163.83 111.665) (end 164.56 112.395) (width 0.3) (layer F.Cu) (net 21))
 (segment (start 142.845 75.945) (end 142.030773 75.945) (width 0.3) (layer F.Cu) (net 22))
 (segment (start 174.72 111.22) (end 174.72 112.395) (width 0.3) (layer F.Cu) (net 22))
 (segment (start 173.355 109.855) (end 174.72 111.22) (width 0.3) (layer F.Cu) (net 22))
 (segment (start 144.24 112.395) (end 144.24 110.395) (width 0.3) (layer F.Cu) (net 23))
 (segment (start 144.24 110.395) (end 144.78 109.855) (width 0.3) (layer F.Cu) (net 23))
 (segment (start 138.43 69.85) (end 140.335 67.945) (width 0.3) (layer F.Cu) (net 25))
 (segment (start 140.335 67.945) (end 142.845 67.945) (width 0.3) (layer F.Cu) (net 25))
 (segment (start 138.43 83.185) (end 138.43 69.85) (width 0.3) (layer F.Cu) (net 25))
 (segment (start 139.7 84.455) (end 138.43 83.185) (width 0.3) (layer F.Cu) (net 25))
 (segment (start 140.335 84.455) (end 139.7 84.455) (width 0.3) (layer F.Cu) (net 25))
 (segment (start 140.335 85.305) (end 140.335 84.455) (width 0.3) (layer F.Cu) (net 25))
 (segment (start 140.875 86.995) (end 140.875 85.845) (width 0.3) (layer F.Cu) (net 25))
 (segment (start 140.875 85.845) (end 140.335 85.305) (width 0.3) (layer F.Cu) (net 25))
 (segment (start 141.025 90.17) (end 142.325001 88.869999) (width 0.3) (layer F.Cu) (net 26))
 (segment (start 142.325001 88.869999) (end 142.325001 84.239228) (width 0.3) (layer F.Cu) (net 26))
 (segment (start 142.325001 84.239228) (end 141.270773 83.185) (width 0.3) (layer F.Cu) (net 26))
 (segment (start 139.7 83.185) (end 139.065 82.55) (width 0.3) (layer F.Cu) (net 26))
 (segment (start 139.065 82.55) (end 139.065 73.66) (width 0.3) (layer F.Cu) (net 26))
 (segment (start 141.270773 83.185) (end 139.7 83.185) (width 0.3) (layer F.Cu) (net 26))
 (segment (start 139.065 73.66) (end 140.78 71.945) (width 0.3) (layer F.Cu) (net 26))
 (segment (start 140.78 71.945) (end 142.845 71.945) (width 0.3) (layer F.Cu) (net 26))
 (segment (start 153.975 92.075) (end 161.925 92.075) (width 0.3) (layer F.Cu) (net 26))
 (segment (start 142.24 92.075) (end 142.24 91.385) (width 0.3) (layer F.Cu) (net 26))
 (segment (start 142.24 91.385) (end 141.025 90.17) (width 0.3) (layer F.Cu) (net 26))
 (segment (start 141.025 90.17) (end 140.875 90.17) (width 0.3) (layer F.Cu) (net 26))
 (segment (start 154.14 107.025) (end 162.09 107.025) (width 0.3) (layer F.Cu) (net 27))
 (segment (start 166.37 80.645) (end 166.37 78.2) (width 0.3) (layer F.Cu) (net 27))
 (segment (start 166.37 78.2) (end 166.275 78.105) (width 0.3) (layer F.Cu) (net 27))
 (via (at 166.37 80.645) (size 0.6) (drill 0.4) (layers F.Cu B.Cu) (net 27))
 (via (at 166.37 90.17) (size 0.6) (drill 0.4) (layers F.Cu B.Cu) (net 27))
 (segment (start 162.09 107.025) (end 162.215 107.025) (width 0.3) (layer F.Cu) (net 27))
 (segment (start 166.275 78.105) (end 164.975 78.105) (width 0.3) (layer F.Cu) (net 27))
 (segment (start 164.975 78.105) (end 162.815 75.945) (width 0.3) (layer F.Cu) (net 27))
 (segment (start 162.815 75.945) (end 156.845 75.945) (width 0.3) (layer F.Cu) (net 27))
 (segment (start 161.925 81.185) (end 160.775 81.185) (width 0.3) (layer F.Cu) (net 28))
 (segment (start 160.775 81.185) (end 159.535 79.945) (width 0.3) (layer F.Cu) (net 28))
 (segment (start 159.535 79.945) (end 156.845 79.945) (width 0.3) (layer F.Cu) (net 28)))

